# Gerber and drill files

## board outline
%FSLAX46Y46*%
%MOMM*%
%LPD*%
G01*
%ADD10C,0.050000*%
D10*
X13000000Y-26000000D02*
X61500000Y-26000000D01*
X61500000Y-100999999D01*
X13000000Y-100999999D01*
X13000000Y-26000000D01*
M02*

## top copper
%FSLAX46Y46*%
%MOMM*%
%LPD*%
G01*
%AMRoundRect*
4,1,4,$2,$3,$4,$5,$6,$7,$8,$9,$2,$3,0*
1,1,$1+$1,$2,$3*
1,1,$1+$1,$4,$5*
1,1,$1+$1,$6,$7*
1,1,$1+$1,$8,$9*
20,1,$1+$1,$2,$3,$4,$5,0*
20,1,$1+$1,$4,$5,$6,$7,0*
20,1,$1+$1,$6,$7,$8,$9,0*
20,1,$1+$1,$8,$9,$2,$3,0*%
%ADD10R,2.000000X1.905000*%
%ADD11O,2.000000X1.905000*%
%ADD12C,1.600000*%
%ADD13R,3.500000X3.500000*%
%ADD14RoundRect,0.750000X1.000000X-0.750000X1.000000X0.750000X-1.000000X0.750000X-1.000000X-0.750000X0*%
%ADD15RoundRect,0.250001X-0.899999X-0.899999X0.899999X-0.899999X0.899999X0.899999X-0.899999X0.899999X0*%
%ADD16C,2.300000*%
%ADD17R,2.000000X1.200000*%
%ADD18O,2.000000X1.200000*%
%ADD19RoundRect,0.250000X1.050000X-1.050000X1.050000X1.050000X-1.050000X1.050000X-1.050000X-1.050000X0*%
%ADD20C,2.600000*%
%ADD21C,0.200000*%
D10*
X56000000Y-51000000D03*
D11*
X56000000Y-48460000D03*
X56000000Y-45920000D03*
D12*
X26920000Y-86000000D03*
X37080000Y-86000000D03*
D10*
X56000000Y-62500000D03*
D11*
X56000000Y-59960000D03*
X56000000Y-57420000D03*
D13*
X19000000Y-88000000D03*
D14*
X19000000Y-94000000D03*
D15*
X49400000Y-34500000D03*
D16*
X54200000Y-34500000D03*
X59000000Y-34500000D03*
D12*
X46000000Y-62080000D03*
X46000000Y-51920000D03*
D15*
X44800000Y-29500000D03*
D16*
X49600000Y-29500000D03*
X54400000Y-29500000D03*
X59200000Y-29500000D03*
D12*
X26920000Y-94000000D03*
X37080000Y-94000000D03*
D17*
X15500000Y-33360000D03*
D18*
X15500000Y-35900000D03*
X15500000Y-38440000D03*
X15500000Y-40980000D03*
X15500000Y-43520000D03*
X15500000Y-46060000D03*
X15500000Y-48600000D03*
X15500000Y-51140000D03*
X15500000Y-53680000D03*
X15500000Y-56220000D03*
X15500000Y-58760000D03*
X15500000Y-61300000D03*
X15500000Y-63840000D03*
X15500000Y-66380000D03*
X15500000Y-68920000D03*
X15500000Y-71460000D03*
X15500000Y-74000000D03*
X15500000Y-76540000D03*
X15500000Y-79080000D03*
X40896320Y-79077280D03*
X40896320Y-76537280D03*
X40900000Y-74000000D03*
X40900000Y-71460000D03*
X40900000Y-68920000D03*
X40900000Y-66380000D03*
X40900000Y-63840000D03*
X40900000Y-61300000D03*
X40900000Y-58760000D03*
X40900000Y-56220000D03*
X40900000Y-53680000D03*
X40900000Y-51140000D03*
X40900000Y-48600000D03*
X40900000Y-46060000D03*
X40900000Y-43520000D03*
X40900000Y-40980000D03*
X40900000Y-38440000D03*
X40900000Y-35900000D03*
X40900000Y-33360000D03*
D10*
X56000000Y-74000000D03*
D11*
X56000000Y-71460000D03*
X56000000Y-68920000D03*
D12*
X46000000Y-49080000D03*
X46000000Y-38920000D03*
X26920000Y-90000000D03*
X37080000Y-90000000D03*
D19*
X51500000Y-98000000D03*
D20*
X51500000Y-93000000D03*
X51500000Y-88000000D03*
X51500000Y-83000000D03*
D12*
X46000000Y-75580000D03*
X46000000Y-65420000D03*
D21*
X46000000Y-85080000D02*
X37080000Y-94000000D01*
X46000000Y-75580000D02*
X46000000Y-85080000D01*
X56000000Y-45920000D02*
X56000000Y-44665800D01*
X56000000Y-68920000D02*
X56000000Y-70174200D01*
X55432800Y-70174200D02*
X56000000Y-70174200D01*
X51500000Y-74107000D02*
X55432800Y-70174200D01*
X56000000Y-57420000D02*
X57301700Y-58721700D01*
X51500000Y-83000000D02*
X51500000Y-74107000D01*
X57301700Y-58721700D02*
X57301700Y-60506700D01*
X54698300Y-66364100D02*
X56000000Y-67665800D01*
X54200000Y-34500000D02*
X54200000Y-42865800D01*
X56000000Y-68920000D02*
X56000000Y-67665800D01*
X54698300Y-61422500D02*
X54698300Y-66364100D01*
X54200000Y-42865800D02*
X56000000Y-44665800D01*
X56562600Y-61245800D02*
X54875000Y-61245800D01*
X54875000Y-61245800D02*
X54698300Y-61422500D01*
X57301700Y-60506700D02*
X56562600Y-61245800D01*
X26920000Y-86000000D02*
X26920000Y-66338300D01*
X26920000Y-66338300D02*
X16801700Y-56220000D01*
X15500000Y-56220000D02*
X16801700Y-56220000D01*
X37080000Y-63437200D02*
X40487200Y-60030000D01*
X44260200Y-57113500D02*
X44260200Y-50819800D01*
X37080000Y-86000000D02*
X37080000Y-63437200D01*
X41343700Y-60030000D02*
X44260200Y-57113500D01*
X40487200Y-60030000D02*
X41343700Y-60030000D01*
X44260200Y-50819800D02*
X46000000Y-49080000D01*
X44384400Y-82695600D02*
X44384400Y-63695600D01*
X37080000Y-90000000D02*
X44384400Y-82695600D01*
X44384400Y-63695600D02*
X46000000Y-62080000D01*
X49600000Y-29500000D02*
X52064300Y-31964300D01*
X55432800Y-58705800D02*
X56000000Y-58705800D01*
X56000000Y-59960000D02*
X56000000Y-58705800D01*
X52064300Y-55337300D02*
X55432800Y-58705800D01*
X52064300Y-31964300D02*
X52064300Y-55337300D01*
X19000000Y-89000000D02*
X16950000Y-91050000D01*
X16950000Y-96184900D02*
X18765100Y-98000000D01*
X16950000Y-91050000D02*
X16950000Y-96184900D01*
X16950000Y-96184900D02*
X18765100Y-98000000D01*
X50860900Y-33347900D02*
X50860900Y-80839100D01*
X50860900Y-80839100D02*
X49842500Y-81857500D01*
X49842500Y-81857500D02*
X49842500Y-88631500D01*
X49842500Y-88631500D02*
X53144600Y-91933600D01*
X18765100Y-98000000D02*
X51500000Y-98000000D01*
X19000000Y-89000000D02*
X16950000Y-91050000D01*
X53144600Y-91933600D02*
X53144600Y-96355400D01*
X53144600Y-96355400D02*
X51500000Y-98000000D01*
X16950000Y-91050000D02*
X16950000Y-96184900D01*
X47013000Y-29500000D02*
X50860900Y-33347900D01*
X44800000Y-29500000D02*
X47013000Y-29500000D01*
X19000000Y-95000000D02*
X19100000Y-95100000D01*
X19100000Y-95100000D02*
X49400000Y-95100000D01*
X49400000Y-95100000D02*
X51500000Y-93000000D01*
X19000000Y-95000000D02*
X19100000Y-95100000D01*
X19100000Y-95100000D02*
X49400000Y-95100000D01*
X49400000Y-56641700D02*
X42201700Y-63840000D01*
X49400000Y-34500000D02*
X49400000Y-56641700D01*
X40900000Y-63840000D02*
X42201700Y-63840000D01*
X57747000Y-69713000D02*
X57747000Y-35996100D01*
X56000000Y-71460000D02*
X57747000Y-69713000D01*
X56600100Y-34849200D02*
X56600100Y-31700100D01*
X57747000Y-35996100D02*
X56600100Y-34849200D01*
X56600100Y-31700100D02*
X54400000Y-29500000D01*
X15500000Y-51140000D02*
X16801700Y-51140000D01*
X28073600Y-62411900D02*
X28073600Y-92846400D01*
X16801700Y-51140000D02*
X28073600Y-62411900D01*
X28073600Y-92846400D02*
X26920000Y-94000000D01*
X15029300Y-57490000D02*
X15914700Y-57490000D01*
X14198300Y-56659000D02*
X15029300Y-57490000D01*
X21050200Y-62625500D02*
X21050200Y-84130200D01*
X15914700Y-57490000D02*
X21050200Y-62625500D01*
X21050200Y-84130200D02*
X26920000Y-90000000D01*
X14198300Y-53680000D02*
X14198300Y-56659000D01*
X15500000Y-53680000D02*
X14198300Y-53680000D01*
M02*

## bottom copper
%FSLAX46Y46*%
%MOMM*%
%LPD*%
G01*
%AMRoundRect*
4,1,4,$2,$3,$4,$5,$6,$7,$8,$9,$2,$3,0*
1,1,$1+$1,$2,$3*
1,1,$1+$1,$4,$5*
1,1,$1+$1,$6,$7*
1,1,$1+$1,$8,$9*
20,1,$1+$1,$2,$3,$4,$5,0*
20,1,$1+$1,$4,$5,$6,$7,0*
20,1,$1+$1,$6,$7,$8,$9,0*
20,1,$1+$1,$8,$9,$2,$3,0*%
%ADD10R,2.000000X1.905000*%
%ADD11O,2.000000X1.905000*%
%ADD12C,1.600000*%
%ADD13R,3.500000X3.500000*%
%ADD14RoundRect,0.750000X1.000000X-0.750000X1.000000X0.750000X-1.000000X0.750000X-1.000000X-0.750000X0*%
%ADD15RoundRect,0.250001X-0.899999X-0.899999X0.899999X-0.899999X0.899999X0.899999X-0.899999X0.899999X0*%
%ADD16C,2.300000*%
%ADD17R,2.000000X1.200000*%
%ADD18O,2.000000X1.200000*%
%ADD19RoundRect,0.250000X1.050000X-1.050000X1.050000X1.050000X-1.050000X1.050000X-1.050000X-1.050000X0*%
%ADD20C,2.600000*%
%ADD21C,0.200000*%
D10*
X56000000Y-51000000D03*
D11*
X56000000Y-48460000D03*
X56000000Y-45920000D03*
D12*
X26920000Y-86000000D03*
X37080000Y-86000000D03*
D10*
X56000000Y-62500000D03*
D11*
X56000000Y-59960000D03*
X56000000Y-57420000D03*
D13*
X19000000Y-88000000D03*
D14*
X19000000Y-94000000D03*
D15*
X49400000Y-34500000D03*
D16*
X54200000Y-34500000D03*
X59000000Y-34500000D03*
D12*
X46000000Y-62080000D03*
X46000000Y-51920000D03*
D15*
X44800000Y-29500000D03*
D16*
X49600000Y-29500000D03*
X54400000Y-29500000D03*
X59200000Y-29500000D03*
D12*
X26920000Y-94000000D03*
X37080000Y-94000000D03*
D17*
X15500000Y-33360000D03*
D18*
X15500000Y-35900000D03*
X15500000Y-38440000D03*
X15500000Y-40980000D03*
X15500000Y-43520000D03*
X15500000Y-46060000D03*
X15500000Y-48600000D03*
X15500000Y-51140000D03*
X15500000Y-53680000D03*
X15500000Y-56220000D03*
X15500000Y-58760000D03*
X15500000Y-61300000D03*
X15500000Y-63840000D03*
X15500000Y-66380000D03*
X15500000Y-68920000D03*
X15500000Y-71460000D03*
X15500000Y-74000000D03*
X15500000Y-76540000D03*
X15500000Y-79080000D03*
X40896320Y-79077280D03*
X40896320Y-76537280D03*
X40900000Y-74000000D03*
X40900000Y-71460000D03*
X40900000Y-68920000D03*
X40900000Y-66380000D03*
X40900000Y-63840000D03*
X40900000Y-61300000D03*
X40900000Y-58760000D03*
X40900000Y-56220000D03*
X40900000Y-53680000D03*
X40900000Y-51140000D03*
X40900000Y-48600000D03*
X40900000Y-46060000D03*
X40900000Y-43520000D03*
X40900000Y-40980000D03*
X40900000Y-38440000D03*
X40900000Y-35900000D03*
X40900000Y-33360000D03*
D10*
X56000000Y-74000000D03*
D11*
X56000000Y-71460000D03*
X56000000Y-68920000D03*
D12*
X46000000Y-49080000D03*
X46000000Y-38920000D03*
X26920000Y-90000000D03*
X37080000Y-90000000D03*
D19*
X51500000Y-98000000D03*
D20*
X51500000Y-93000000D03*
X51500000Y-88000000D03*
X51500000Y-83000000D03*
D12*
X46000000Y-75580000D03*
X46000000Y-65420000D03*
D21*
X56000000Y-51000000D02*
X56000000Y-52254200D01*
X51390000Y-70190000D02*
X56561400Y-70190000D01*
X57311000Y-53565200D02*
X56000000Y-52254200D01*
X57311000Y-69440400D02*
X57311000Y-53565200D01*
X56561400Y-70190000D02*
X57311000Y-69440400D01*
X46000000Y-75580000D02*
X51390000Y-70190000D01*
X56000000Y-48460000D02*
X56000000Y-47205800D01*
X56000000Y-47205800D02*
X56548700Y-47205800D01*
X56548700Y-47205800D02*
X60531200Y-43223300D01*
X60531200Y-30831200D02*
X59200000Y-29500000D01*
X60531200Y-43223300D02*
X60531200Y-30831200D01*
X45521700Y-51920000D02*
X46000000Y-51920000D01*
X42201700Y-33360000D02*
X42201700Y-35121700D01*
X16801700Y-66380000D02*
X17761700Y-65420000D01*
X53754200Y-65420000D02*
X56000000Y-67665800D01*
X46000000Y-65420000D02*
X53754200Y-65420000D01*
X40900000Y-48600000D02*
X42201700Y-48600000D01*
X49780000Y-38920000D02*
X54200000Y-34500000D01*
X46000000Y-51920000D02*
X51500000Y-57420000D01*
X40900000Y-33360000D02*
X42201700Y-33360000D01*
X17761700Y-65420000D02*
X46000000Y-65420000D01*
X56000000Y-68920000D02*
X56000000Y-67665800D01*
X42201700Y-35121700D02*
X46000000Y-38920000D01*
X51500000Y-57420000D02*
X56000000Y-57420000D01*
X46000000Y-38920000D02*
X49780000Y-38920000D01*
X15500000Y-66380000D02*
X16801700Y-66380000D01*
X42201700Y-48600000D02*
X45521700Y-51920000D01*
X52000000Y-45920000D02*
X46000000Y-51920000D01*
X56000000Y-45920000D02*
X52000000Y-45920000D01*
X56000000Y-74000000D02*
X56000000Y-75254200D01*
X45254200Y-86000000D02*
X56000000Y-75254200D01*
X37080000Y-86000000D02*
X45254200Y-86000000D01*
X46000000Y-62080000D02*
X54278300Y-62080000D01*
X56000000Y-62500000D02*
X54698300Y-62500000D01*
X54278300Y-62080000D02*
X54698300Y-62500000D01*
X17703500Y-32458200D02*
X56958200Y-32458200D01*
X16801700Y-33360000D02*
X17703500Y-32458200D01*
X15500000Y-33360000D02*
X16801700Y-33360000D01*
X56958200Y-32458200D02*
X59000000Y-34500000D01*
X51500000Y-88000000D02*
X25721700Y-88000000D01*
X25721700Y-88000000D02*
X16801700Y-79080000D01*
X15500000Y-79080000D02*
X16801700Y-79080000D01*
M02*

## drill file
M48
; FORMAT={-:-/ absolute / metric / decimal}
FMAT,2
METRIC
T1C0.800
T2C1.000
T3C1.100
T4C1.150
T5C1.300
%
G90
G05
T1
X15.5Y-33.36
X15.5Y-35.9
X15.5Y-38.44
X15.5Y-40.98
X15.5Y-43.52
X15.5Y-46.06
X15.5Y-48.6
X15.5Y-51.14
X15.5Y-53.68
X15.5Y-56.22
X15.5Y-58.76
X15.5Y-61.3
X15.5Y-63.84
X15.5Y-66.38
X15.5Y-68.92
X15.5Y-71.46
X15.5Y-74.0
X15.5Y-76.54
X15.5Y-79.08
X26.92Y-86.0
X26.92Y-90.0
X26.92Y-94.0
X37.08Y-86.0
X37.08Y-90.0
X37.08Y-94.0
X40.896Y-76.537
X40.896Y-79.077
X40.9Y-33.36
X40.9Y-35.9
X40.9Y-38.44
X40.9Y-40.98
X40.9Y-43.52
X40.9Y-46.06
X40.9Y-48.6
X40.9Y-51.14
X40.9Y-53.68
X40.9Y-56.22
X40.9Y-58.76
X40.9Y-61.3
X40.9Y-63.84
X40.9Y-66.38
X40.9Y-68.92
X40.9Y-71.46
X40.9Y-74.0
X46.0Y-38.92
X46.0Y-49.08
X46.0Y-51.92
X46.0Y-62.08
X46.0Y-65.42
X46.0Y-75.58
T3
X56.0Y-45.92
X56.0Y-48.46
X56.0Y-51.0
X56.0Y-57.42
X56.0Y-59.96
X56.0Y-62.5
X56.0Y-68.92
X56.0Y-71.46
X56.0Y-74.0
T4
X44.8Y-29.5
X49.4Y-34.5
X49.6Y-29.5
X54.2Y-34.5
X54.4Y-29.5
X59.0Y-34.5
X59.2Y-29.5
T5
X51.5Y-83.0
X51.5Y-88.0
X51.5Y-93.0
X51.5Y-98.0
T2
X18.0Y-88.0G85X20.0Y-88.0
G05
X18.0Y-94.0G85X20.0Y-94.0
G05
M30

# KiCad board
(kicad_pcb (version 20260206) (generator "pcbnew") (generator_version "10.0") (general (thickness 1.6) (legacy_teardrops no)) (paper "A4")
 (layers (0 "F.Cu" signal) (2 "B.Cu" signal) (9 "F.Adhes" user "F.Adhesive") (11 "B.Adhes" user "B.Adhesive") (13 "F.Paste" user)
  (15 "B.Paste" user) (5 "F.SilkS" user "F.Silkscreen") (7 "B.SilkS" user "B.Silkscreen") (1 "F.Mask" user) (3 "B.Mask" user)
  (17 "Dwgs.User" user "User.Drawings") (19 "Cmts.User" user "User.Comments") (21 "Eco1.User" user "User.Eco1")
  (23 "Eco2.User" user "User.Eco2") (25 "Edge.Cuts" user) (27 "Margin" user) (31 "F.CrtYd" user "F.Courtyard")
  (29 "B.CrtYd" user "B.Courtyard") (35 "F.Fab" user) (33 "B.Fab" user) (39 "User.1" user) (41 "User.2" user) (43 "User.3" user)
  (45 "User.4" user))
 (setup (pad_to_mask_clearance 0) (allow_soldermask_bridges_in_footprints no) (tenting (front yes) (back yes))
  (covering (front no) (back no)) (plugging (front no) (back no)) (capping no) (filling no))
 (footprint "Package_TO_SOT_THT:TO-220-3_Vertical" (layer "F.Cu") (at 56 51 90)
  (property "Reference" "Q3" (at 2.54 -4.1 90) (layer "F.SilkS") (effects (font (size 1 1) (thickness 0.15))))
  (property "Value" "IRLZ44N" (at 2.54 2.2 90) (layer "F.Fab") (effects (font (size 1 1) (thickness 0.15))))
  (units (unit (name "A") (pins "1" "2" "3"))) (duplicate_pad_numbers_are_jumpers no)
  (pad "1" thru_hole rect (at 0 0 90) (size 1.905 2) (drill 1.1) (layers "*.Cu" "*.Mask") (remove_unused_layers no) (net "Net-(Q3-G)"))
  (pad "2" thru_hole oval (at 2.54 0 90) (size 1.905 2) (drill 1.1) (layers "*.Cu" "*.Mask") (remove_unused_layers no) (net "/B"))
  (pad "3" thru_hole oval (at 5.08 0 90) (size 1.905 2) (drill 1.1) (layers "*.Cu" "*.Mask") (remove_unused_layers no) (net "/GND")))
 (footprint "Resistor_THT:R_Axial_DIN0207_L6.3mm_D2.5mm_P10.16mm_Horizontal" (layer "F.Cu") (at 26.92 86)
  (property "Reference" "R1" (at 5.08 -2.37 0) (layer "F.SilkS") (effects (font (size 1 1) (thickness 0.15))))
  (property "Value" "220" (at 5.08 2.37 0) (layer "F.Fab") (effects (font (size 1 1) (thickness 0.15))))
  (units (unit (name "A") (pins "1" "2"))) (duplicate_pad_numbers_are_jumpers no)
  (pad "1" thru_hole circle (at 0 0) (size 1.6 1.6) (drill 0.8) (layers "*.Cu" "*.Mask") (remove_unused_layers no)
   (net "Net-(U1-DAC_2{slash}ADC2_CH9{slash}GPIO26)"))
  (pad "2" thru_hole circle (at 10.16 0) (size 1.6 1.6) (drill 0.8) (layers "*.Cu" "*.Mask") (remove_unused_layers no) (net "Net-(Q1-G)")))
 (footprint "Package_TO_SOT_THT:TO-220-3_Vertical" (layer "F.Cu") (at 56 62.5 90)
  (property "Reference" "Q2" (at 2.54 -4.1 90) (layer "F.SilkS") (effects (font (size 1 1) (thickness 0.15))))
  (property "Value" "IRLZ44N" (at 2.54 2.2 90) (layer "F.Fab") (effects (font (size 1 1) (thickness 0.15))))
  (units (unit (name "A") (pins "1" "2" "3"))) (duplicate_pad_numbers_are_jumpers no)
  (pad "1" thru_hole rect (at 0 0 90) (size 1.905 2) (drill 1.1) (layers "*.Cu" "*.Mask") (remove_unused_layers no) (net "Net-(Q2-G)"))
  (pad "2" thru_hole oval (at 2.54 0 90) (size 1.905 2) (drill 1.1) (layers "*.Cu" "*.Mask") (remove_unused_layers no) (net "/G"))
  (pad "3" thru_hole oval (at 5.08 0 90) (size 1.905 2) (drill 1.1) (layers "*.Cu" "*.Mask") (remove_unused_layers no) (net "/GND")))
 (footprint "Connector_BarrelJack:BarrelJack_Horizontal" (layer "F.Cu") (at 19 88 90)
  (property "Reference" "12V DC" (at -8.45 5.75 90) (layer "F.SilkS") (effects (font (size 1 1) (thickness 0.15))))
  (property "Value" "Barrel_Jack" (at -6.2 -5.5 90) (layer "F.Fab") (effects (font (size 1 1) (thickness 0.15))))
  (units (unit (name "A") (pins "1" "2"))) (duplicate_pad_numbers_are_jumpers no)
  (pad "1" thru_hole rect (at 0 0 90) (size 3.5 3.5) (drill oval 1 3) (layers "*.Cu" "*.Mask") (remove_unused_layers no) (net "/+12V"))
  (pad "2" thru_hole roundrect (at -6 0 90) (size 3 3.5) (drill oval 1 3) (layers "*.Cu" "*.Mask") (remove_unused_layers no)
   (roundrect_rratio 0.25) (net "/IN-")))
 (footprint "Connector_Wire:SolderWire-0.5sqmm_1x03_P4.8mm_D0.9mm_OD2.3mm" (layer "F.Cu") (at 49.4 34.5)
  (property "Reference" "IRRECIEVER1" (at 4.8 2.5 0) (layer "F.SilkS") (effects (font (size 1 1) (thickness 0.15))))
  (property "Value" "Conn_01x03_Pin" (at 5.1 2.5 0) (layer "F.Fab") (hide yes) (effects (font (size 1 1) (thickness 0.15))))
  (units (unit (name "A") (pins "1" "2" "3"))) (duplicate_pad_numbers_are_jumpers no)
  (pad "1" thru_hole roundrect (at 0 0) (size 2.3 2.3) (drill 1.15) (layers "*.Cu" "*.Mask") (remove_unused_layers no)
   (roundrect_rratio 0.108696) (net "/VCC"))
  (pad "2" thru_hole circle (at 4.8 0) (size 2.3 2.3) (drill 1.15) (layers "*.Cu" "*.Mask") (remove_unused_layers no) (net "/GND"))
  (pad "3" thru_hole circle (at 9.6 0) (size 2.3 2.3) (drill 1.15) (layers "*.Cu" "*.Mask") (remove_unused_layers no) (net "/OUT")))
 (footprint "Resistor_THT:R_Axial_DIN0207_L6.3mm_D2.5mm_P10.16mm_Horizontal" (layer "F.Cu") (at 46 62.08 90)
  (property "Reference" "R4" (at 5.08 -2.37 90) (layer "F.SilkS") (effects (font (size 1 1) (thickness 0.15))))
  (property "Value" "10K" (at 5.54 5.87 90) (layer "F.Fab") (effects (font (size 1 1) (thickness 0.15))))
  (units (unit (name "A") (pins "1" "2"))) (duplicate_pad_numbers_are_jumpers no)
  (pad "1" thru_hole circle (at 0 0 90) (size 1.6 1.6) (drill 0.8) (layers "*.Cu" "*.Mask") (remove_unused_layers no) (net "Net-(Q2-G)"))
  (pad "2" thru_hole circle (at 10.16 0 90) (size 1.6 1.6) (drill 0.8) (layers "*.Cu" "*.Mask") (remove_unused_layers no) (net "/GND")))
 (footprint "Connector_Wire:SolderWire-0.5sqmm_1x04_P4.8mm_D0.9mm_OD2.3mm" (layer "F.Cu") (at 44.8 29.5)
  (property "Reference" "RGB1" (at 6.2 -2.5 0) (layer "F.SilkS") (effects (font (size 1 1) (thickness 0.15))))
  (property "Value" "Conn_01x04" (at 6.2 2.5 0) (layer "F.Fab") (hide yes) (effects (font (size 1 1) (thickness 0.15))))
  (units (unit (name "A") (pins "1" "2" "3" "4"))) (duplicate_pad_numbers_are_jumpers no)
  (pad "1" thru_hole roundrect (at 0 0) (size 2.3 2.3) (drill 1.15) (layers "*.Cu" "*.Mask") (remove_unused_layers no)
   (roundrect_rratio 0.108696) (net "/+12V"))
  (pad "2" thru_hole circle (at 4.8 0) (size 2.3 2.3) (drill 1.15) (layers "*.Cu" "*.Mask") (remove_unused_layers no) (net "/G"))
  (pad "3" thru_hole circle (at 9.6 0) (size 2.3 2.3) (drill 1.15) (layers "*.Cu" "*.Mask") (remove_unused_layers no) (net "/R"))
  (pad "4" thru_hole circle (at 14.4 0) (size 2.3 2.3) (drill 1.15) (layers "*.Cu" "*.Mask") (remove_unused_layers no) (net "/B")))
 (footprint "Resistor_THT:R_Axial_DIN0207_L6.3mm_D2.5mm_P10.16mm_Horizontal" (layer "F.Cu") (at 26.92 94)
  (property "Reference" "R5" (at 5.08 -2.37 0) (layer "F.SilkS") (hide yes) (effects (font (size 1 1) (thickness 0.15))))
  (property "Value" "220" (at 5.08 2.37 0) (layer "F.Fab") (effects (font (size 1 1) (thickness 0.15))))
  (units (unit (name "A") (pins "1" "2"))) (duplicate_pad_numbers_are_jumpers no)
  (pad "1" thru_hole circle (at 0 0) (size 1.6 1.6) (drill 0.8) (layers "*.Cu" "*.Mask") (remove_unused_layers no)
   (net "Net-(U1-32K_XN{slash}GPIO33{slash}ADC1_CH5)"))
  (pad "2" thru_hole circle (at 10.16 0) (size 1.6 1.6) (drill 0.8) (layers "*.Cu" "*.Mask") (remove_unused_layers no) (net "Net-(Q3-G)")))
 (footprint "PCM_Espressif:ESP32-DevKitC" (layer "F.Cu") (at 15.5 33.36)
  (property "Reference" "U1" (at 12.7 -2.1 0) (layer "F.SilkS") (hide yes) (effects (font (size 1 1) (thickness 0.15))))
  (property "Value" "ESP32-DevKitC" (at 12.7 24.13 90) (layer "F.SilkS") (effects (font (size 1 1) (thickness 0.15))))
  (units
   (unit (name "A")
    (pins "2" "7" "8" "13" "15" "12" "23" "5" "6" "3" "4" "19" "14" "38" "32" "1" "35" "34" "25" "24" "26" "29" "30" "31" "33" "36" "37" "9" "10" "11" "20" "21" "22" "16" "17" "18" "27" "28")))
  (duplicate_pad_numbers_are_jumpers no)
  (pad "1" thru_hole rect (at 0 0 270) (size 1.2 2) (drill 0.8) (layers "*.Cu" "*.Mask") (remove_unused_layers no) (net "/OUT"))
  (pad "2" thru_hole oval (at 0 2.54 270) (size 1.2 2) (drill 0.8) (layers "*.Cu" "*.Mask") (remove_unused_layers no)
   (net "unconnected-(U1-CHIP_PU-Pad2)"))
  (pad "3" thru_hole oval (at 0 5.08 270) (size 1.2 2) (drill 0.8) (layers "*.Cu" "*.Mask") (remove_unused_layers no)
   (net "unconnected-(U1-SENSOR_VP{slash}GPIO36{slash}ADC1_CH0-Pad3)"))
  (pad "4" thru_hole oval (at 0 7.62 270) (size 1.2 2) (drill 0.8) (layers "*.Cu" "*.Mask") (remove_unused_layers no)
   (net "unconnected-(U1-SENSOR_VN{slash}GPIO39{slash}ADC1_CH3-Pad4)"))
  (pad "5" thru_hole oval (at 0 10.16 270) (size 1.2 2) (drill 0.8) (layers "*.Cu" "*.Mask") (remove_unused_layers no)
   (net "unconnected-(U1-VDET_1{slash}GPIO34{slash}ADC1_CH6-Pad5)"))
  (pad "6" thru_hole oval (at 0 12.7 270) (size 1.2 2) (drill 0.8) (layers "*.Cu" "*.Mask") (remove_unused_layers no)
   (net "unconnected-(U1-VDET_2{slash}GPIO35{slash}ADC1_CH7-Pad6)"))
  (pad "7" thru_hole oval (at 0 15.24 270) (size 1.2 2) (drill 0.8) (layers "*.Cu" "*.Mask") (remove_unused_layers no)
   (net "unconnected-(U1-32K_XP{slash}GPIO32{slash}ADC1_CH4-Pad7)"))
  (pad "8" thru_hole oval (at 0 17.78 270) (size 1.2 2) (drill 0.8) (layers "*.Cu" "*.Mask") (remove_unused_layers no)
   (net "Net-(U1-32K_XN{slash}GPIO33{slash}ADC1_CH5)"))
  (pad "9" thru_hole oval (at 0 20.32 270) (size 1.2 2) (drill 0.8) (layers "*.Cu" "*.Mask") (remove_unused_layers no)
   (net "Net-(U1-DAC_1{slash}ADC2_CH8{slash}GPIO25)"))
  (pad "10" thru_hole oval (at 0 22.86 270) (size 1.2 2) (drill 0.8) (layers "*.Cu" "*.Mask") (remove_unused_layers no)
   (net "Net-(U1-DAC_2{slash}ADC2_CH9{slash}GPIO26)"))
  (pad "11" thru_hole oval (at 0 25.4 270) (size 1.2 2) (drill 0.8) (layers "*.Cu" "*.Mask") (remove_unused_layers no)
   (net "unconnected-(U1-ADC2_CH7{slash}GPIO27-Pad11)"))
  (pad "12" thru_hole oval (at 0 27.94 270) (size 1.2 2) (drill 0.8) (layers "*.Cu" "*.Mask") (remove_unused_layers no)
   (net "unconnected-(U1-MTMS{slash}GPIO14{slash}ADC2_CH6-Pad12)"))
  (pad "13" thru_hole oval (at 0 30.48 270) (size 1.2 2) (drill 0.8) (layers "*.Cu" "*.Mask") (remove_unused_layers no)
   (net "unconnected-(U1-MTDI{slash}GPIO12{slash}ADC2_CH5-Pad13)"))
  (pad "14" thru_hole oval (at 0 33.02 270) (size 1.2 2) (drill 0.8) (layers "*.Cu" "*.Mask") (remove_unused_layers no) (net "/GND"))
  (pad "15" thru_hole oval (at 0 35.56 270) (size 1.2 2) (drill 0.8) (layers "*.Cu" "*.Mask") (remove_unused_layers no)
   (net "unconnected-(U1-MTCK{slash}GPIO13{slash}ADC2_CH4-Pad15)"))
  (pad "16" thru_hole oval (at 0 38.1 270) (size 1.2 2) (drill 0.8) (layers "*.Cu" "*.Mask") (remove_unused_layers no)
   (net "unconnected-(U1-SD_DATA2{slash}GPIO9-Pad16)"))
  (pad "17" thru_hole oval (at 0 40.64 270) (size 1.2 2) (drill 0.8) (layers "*.Cu" "*.Mask") (remove_unused_layers no)
   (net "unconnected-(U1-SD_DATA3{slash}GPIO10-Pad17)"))
  (pad "18" thru_hole oval (at 0 43.18 270) (size 1.2 2) (drill 0.8) (layers "*.Cu" "*.Mask") (remove_unused_layers no)
   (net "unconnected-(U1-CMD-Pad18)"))
  (pad "19" thru_hole oval (at 0 45.72 270) (size 1.2 2) (drill 0.8) (layers "*.Cu" "*.Mask") (remove_unused_layers no) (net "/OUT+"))
  (pad "20" thru_hole oval (at 25.39632 45.71728 270) (size 1.2 2) (drill 0.8) (layers "*.Cu" "*.Mask") (remove_unused_layers no)
   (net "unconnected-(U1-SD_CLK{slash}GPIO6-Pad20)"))
  (pad "21" thru_hole oval (at 25.39632 43.17728 270) (size 1.2 2) (drill 0.8) (layers "*.Cu" "*.Mask") (remove_unused_layers no)
   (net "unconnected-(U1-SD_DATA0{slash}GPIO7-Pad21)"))
  (pad "22" thru_hole oval (at 25.4 40.64 270) (size 1.2 2) (drill 0.8) (layers "*.Cu" "*.Mask") (remove_unused_layers no)
   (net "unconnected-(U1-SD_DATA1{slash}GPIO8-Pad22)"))
  (pad "23" thru_hole oval (at 25.4 38.1 270) (size 1.2 2) (drill 0.8) (layers "*.Cu" "*.Mask") (remove_unused_layers no)
   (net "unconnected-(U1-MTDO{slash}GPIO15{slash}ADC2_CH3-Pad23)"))
  (pad "24" thru_hole oval (at 25.4 35.56 270) (size 1.2 2) (drill 0.8) (layers "*.Cu" "*.Mask") (remove_unused_layers no)
   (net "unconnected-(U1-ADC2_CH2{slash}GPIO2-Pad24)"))
  (pad "25" thru_hole oval (at 25.4 33.02 270) (size 1.2 2) (drill 0.8) (layers "*.Cu" "*.Mask") (remove_unused_layers no)
   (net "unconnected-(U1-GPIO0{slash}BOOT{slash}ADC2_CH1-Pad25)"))
  (pad "26" thru_hole oval (at 25.4 30.48 270) (size 1.2 2) (drill 0.8) (layers "*.Cu" "*.Mask") (remove_unused_layers no) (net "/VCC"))
  (pad "27" thru_hole oval (at 25.4 27.94 270) (size 1.2 2) (drill 0.8) (layers "*.Cu" "*.Mask") (remove_unused_layers no)
   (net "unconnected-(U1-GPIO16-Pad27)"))
  (pad "28" thru_hole oval (at 25.4 25.4 270) (size 1.2 2) (drill 0.8) (layers "*.Cu" "*.Mask") (remove_unused_layers no)
   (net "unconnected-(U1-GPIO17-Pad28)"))
  (pad "29" thru_hole oval (at 25.4 22.86 270) (size 1.2 2) (drill 0.8) (layers "*.Cu" "*.Mask") (remove_unused_layers no)
   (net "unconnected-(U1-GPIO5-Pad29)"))
  (pad "30" thru_hole oval (at 25.4 20.32 270) (size 1.2 2) (drill 0.8) (layers "*.Cu" "*.Mask") (remove_unused_layers no)
   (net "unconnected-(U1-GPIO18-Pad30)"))
  (pad "31" thru_hole oval (at 25.4 17.78 270) (size 1.2 2) (drill 0.8) (layers "*.Cu" "*.Mask") (remove_unused_layers no)
   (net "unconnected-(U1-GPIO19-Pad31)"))
  (pad "32" thru_hole oval (at 25.4 15.24 270) (size 1.2 2) (drill 0.8) (layers "*.Cu" "*.Mask") (remove_unused_layers no) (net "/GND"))
  (pad "33" thru_hole oval (at 25.4 12.7 270) (size 1.2 2) (drill 0.8) (layers "*.Cu" "*.Mask") (remove_unused_layers no)
   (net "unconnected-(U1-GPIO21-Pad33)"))
  (pad "34" thru_hole oval (at 25.4 10.16 270) (size 1.2 2) (drill 0.8) (layers "*.Cu" "*.Mask") (remove_unused_layers no)
   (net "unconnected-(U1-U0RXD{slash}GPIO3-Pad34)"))
  (pad "35" thru_hole oval (at 25.4 7.62 270) (size 1.2 2) (drill 0.8) (layers "*.Cu" "*.Mask") (remove_unused_layers no)
   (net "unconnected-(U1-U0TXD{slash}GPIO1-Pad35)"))
  (pad "36" thru_hole oval (at 25.4 5.08 270) (size 1.2 2) (drill 0.8) (layers "*.Cu" "*.Mask") (remove_unused_layers no)
   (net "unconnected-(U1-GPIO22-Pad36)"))
  (pad "37" thru_hole oval (at 25.4 2.54 270) (size 1.2 2) (drill 0.8) (layers "*.Cu" "*.Mask") (remove_unused_layers no)
   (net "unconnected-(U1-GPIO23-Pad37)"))
  (pad "38" thru_hole oval (at 25.4 0 270) (size 1.2 2) (drill 0.8) (layers "*.Cu" "*.Mask") (remove_unused_layers no) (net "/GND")))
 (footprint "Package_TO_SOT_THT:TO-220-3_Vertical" (layer "F.Cu") (at 56 74 90)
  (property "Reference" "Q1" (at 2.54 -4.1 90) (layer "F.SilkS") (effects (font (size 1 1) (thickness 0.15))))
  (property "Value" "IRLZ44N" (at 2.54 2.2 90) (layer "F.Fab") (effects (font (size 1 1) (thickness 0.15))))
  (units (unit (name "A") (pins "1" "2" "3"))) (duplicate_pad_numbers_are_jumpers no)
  (pad "1" thru_hole rect (at 0 0 90) (size 1.905 2) (drill 1.1) (layers "*.Cu" "*.Mask") (remove_unused_layers no) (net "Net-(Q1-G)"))
  (pad "2" thru_hole oval (at 2.54 0 90) (size 1.905 2) (drill 1.1) (layers "*.Cu" "*.Mask") (remove_unused_layers no) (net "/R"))
  (pad "3" thru_hole oval (at 5.08 0 90) (size 1.905 2) (drill 1.1) (layers "*.Cu" "*.Mask") (remove_unused_layers no) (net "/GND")))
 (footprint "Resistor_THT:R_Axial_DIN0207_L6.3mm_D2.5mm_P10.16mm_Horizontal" (layer "F.Cu") (at 46 49.08 90)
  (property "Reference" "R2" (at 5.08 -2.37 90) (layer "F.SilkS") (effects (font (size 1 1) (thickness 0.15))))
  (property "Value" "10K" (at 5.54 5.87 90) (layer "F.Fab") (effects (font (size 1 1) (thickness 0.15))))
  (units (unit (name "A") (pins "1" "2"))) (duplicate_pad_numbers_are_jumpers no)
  (pad "1" thru_hole circle (at 0 0 90) (size 1.6 1.6) (drill 0.8) (layers "*.Cu" "*.Mask") (remove_unused_layers no) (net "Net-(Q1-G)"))
  (pad "2" thru_hole circle (at 10.16 0 90) (size 1.6 1.6) (drill 0.8) (layers "*.Cu" "*.Mask") (remove_unused_layers no) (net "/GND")))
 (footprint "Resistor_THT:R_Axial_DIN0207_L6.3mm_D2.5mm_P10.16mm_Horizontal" (layer "F.Cu") (at 26.92 90)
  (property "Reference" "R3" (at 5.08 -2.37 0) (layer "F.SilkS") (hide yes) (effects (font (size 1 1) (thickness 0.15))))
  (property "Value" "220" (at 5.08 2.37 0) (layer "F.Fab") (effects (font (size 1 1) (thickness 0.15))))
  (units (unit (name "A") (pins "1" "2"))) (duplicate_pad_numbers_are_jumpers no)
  (pad "1" thru_hole circle (at 0 0) (size 1.6 1.6) (drill 0.8) (layers "*.Cu" "*.Mask") (remove_unused_layers no)
   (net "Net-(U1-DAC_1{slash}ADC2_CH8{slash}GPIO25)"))
  (pad "2" thru_hole circle (at 10.16 0) (size 1.6 1.6) (drill 0.8) (layers "*.Cu" "*.Mask") (remove_unused_layers no) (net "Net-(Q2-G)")))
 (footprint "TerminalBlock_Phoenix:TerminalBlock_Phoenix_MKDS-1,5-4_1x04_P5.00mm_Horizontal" (layer "F.Cu") (at 51.5 98 90)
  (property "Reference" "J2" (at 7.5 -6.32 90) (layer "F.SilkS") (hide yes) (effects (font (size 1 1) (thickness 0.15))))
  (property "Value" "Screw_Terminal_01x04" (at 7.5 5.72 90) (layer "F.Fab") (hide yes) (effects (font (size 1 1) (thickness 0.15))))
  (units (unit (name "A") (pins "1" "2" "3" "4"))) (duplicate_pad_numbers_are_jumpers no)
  (pad "1" thru_hole roundrect (at 0 0 90) (size 2.6 2.6) (drill 1.3) (layers "*.Cu" "*.Mask") (remove_unused_layers no)
   (roundrect_rratio 0.096154) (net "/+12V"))
  (pad "2" thru_hole circle (at 5 0 90) (size 2.6 2.6) (drill 1.3) (layers "*.Cu" "*.Mask") (remove_unused_layers no) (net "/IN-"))
  (pad "3" thru_hole circle (at 10 0 90) (size 2.6 2.6) (drill 1.3) (layers "*.Cu" "*.Mask") (remove_unused_layers no) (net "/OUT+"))
  (pad "4" thru_hole circle (at 15 0 90) (size 2.6 2.6) (drill 1.3) (layers "*.Cu" "*.Mask") (remove_unused_layers no) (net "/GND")))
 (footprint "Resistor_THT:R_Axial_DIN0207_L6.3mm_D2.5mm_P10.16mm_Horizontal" (layer "F.Cu") (at 46 75.58 90)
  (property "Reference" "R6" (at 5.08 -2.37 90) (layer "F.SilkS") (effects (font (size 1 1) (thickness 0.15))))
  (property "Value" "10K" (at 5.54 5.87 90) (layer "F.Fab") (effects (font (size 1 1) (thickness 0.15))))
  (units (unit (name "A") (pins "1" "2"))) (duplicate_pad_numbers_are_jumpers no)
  (pad "1" thru_hole circle (at 0 0 90) (size 1.6 1.6) (drill 0.8) (layers "*.Cu" "*.Mask") (remove_unused_layers no) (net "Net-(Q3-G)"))
  (pad "2" thru_hole circle (at 10.16 0 90) (size 1.6 1.6) (drill 0.8) (layers "*.Cu" "*.Mask") (remove_unused_layers no) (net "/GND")))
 (gr_rect (start 13 26) (end 61.5 100.999999) (stroke (width 0.05) (type default)) (fill no) (layer "Edge.Cuts"))
 (segment (start 46 85.08) (end 37.08 94) (width 0.2) (layer "F.Cu") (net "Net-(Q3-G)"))
 (segment (start 46 75.58) (end 46 85.08) (width 0.2) (layer "F.Cu") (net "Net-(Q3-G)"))
 (segment (start 56 51) (end 56 52.2542) (width 0.2) (layer "B.Cu") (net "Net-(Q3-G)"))
 (segment (start 51.39 70.19) (end 56.5614 70.19) (width 0.2) (layer "B.Cu") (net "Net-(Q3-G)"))
 (segment (start 57.311 53.5652) (end 56 52.2542) (width 0.2) (layer "B.Cu") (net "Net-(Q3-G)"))
 (segment (start 57.311 69.4404) (end 57.311 53.5652) (width 0.2) (layer "B.Cu") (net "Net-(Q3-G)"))
 (segment (start 56.5614 70.19) (end 57.311 69.4404) (width 0.2) (layer "B.Cu") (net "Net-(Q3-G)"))
 (segment (start 46 75.58) (end 51.39 70.19) (width 0.2) (layer "B.Cu") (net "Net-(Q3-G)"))
 (segment (start 56 48.46) (end 56 47.2058) (width 0.2) (layer "B.Cu") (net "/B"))
 (segment (start 56 47.2058) (end 56.5487 47.2058) (width 0.2) (layer "B.Cu") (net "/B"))
 (segment (start 56.5487 47.2058) (end 60.5312 43.2233) (width 0.2) (layer "B.Cu") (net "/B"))
 (segment (start 60.5312 30.8312) (end 59.2 29.5) (width 0.2) (layer "B.Cu") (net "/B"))
 (segment (start 60.5312 43.2233) (end 60.5312 30.8312) (width 0.2) (layer "B.Cu") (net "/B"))
 (segment (start 56 45.92) (end 56 44.6658) (width 0.2) (layer "F.Cu") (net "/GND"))
 (segment (start 56 68.92) (end 56 70.1742) (width 0.2) (layer "F.Cu") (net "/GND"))
 (segment (start 55.4328 70.1742) (end 56 70.1742) (width 0.2) (layer "F.Cu") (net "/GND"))
 (segment (start 51.5 74.107) (end 55.4328 70.1742) (width 0.2) (layer "F.Cu") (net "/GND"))
 (segment (start 56 57.42) (end 57.3017 58.7217) (width 0.2) (layer "F.Cu") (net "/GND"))
 (segment (start 51.5 83) (end 51.5 74.107) (width 0.2) (layer "F.Cu") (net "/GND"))
 (segment (start 57.3017 58.7217) (end 57.3017 60.5067) (width 0.2) (layer "F.Cu") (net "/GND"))
 (segment (start 54.6983 66.3641) (end 56 67.6658) (width 0.2) (layer "F.Cu") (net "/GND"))
 (segment (start 54.2 34.5) (end 54.2 42.8658) (width 0.2) (layer "F.Cu") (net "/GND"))
 (segment (start 56 68.92) (end 56 67.6658) (width 0.2) (layer "F.Cu") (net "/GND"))
 (segment (start 54.6983 61.4225) (end 54.6983 66.3641) (width 0.2) (layer "F.Cu") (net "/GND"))
 (segment (start 54.2 42.8658) (end 56 44.6658) (width 0.2) (layer "F.Cu") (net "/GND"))
 (segment (start 56.5626 61.2458) (end 54.875 61.2458) (width 0.2) (layer "F.Cu") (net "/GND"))
 (segment (start 54.875 61.2458) (end 54.6983 61.4225) (width 0.2) (layer "F.Cu") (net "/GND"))
 (segment (start 57.3017 60.5067) (end 56.5626 61.2458) (width 0.2) (layer "F.Cu") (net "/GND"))
 (segment (start 45.5217 51.92) (end 46 51.92) (width 0.2) (layer "B.Cu") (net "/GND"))
 (segment (start 42.2017 33.36) (end 42.2017 35.1217) (width 0.2) (layer "B.Cu") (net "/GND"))
 (segment (start 16.8017 66.38) (end 17.7617 65.42) (width 0.2) (layer "B.Cu") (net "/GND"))
 (segment (start 53.7542 65.42) (end 56 67.6658) (width 0.2) (layer "B.Cu") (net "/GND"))
 (segment (start 46 65.42) (end 53.7542 65.42) (width 0.2) (layer "B.Cu") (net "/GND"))
 (segment (start 40.9 48.6) (end 42.2017 48.6) (width 0.2) (layer "B.Cu") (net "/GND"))
 (segment (start 49.78 38.92) (end 54.2 34.5) (width 0.2) (layer "B.Cu") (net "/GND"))
 (segment (start 46 51.92) (end 51.5 57.42) (width 0.2) (layer "B.Cu") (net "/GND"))
 (segment (start 40.9 33.36) (end 42.2017 33.36) (width 0.2) (layer "B.Cu") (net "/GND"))
 (segment (start 17.7617 65.42) (end 46 65.42) (width 0.2) (layer "B.Cu") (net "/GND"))
 (segment (start 56 68.92) (end 56 67.6658) (width 0.2) (layer "B.Cu") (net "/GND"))
 (segment (start 42.2017 35.1217) (end 46 38.92) (width 0.2) (layer "B.Cu") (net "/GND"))
 (segment (start 51.5 57.42) (end 56 57.42) (width 0.2) (layer "B.Cu") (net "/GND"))
 (segment (start 46 38.92) (end 49.78 38.92) (width 0.2) (layer "B.Cu") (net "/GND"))
 (segment (start 15.5 66.38) (end 16.8017 66.38) (width 0.2) (layer "B.Cu") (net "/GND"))
 (segment (start 42.2017 48.6) (end 45.5217 51.92) (width 0.2) (layer "B.Cu") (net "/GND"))
 (segment (start 52 45.92) (end 46 51.92) (width 0.2) (layer "B.Cu") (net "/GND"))
 (segment (start 56 45.92) (end 52 45.92) (width 0.2) (layer "B.Cu") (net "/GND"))
 (segment (start 26.92 86) (end 26.92 66.3383) (width 0.2) (layer "F.Cu") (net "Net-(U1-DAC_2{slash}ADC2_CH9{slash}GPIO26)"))
 (segment (start 26.92 66.3383) (end 16.8017 56.22) (width 0.2) (layer "F.Cu") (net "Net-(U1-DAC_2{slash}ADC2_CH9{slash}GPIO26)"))
 (segment (start 15.5 56.22) (end 16.8017 56.22) (width 0.2) (layer "F.Cu") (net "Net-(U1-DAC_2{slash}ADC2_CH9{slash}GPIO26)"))
 (segment (start 37.08 63.4372) (end 40.4872 60.03) (width 0.2) (layer "F.Cu") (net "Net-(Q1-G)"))
 (segment (start 44.2602 57.1135) (end 44.2602 50.8198) (width 0.2) (layer "F.Cu") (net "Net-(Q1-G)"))
 (segment (start 37.08 86) (end 37.08 63.4372) (width 0.2) (layer "F.Cu") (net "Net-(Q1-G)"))
 (segment (start 41.3437 60.03) (end 44.2602 57.1135) (width 0.2) (layer "F.Cu") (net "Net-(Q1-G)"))
 (segment (start 40.4872 60.03) (end 41.3437 60.03) (width 0.2) (layer "F.Cu") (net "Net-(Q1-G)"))
 (segment (start 44.2602 50.8198) (end 46 49.08) (width 0.2) (layer "F.Cu") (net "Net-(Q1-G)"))
 (segment (start 56 74) (end 56 75.2542) (width 0.2) (layer "B.Cu") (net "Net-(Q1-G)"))
 (segment (start 45.2542 86) (end 56 75.2542) (width 0.2) (layer "B.Cu") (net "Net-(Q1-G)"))
 (segment (start 37.08 86) (end 45.2542 86) (width 0.2) (layer "B.Cu") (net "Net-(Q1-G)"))
 (segment (start 44.3844 82.6956) (end 44.3844 63.6956) (width 0.2) (layer "F.Cu") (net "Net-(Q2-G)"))
 (segment (start 37.08 90) (end 44.3844 82.6956) (width 0.2) (layer "F.Cu") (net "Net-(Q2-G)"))
 (segment (start 44.3844 63.6956) (end 46 62.08) (width 0.2) (layer "F.Cu") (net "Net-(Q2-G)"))
 (segment (start 46 62.08) (end 54.2783 62.08) (width 0.2) (layer "B.Cu") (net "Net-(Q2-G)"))
 (segment (start 56 62.5) (end 54.6983 62.5) (width 0.2) (layer "B.Cu") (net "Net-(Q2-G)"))
 (segment (start 54.2783 62.08) (end 54.6983 62.5) (width 0.2) (layer "B.Cu") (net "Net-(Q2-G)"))
 (segment (start 49.6 29.5) (end 52.0643 31.9643) (width 0.2) (layer "F.Cu") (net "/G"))
 (segment (start 55.4328 58.7058) (end 56 58.7058) (width 0.2) (layer "F.Cu") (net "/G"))
 (segment (start 56 59.96) (end 56 58.7058) (width 0.2) (layer "F.Cu") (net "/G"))
 (segment (start 52.0643 55.3373) (end 55.4328 58.7058) (width 0.2) (layer "F.Cu") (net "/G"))
 (segment (start 52.0643 31.9643) (end 52.0643 55.3373) (width 0.2) (layer "F.Cu") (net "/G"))
 (segment (start 19 89) (end 16.95 91.05) (width 0.2) (layer "F.Cu") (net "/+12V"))
 (segment (start 16.95 96.1849) (end 18.7651 98) (width 0.2) (layer "F.Cu") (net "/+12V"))
 (segment (start 16.95 91.05) (end 16.95 96.1849) (width 0.2) (layer "F.Cu") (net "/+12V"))
 (segment (start 16.95 96.1849) (end 18.7651 98) (width 0.2) (layer "F.Cu") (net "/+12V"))
 (segment (start 50.8609 33.3479) (end 50.8609 80.8391) (width 0.2) (layer "F.Cu") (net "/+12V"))
 (segment (start 50.8609 80.8391) (end 49.8425 81.8575) (width 0.2) (layer "F.Cu") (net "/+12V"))
 (segment (start 49.8425 81.8575) (end 49.8425 88.6315) (width 0.2) (layer "F.Cu") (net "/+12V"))
 (segment (start 49.8425 88.6315) (end 53.1446 91.9336) (width 0.2) (layer "F.Cu") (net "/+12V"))
 (segment (start 18.7651 98) (end 51.5 98) (width 0.2) (layer "F.Cu") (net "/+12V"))
 (segment (start 19 89) (end 16.95 91.05) (width 0.2) (layer "F.Cu") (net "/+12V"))
 (segment (start 53.1446 91.9336) (end 53.1446 96.3554) (width 0.2) (layer "F.Cu") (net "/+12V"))
 (segment (start 53.1446 96.3554) (end 51.5 98) (width 0.2) (layer "F.Cu") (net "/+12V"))
 (segment (start 16.95 91.05) (end 16.95 96.1849) (width 0.2) (layer "F.Cu") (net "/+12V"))
 (segment (start 47.013 29.5) (end 50.8609 33.3479) (width 0.2) (layer "F.Cu") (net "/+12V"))
 (segment (start 44.8 29.5) (end 47.013 29.5) (width 0.2) (layer "F.Cu") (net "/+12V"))
 (segment (start 19 95) (end 19.1 95.1) (width 0.2) (layer "F.Cu") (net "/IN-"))
 (segment (start 19.1 95.1) (end 49.4 95.1) (width 0.2) (layer "F.Cu") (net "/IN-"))
 (segment (start 49.4 95.1) (end 51.5 93) (width 0.2) (layer "F.Cu") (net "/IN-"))
 (segment (start 19 95) (end 19.1 95.1) (width 0.2) (layer "F.Cu") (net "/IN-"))
 (segment (start 19.1 95.1) (end 49.4 95.1) (width 0.2) (layer "F.Cu") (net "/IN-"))
 (segment (start 49.4 56.6417) (end 42.2017 63.84) (width 0.2) (layer "F.Cu") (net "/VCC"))
 (segment (start 49.4 34.5) (end 49.4 56.6417) (width 0.2) (layer "F.Cu") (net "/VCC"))
 (segment (start 40.9 63.84) (end 42.2017 63.84) (width 0.2) (layer "F.Cu") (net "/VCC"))
 (segment (start 17.7035 32.4582) (end 56.9582 32.4582) (width 0.2) (layer "B.Cu") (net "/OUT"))
 (segment (start 16.8017 33.36) (end 17.7035 32.4582) (width 0.2) (layer "B.Cu") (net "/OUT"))
 (segment (start 15.5 33.36) (end 16.8017 33.36) (width 0.2) (layer "B.Cu") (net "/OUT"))
 (segment (start 56.9582 32.4582) (end 59 34.5) (width 0.2) (layer "B.Cu") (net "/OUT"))
 (segment (start 57.747 69.713) (end 57.747 35.9961) (width 0.2) (layer "F.Cu") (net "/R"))
 (segment (start 56 71.46) (end 57.747 69.713) (width 0.2) (layer "F.Cu") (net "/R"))
 (segment (start 56.6001 34.8492) (end 56.6001 31.7001) (width 0.2) (layer "F.Cu") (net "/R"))
 (segment (start 57.747 35.9961) (end 56.6001 34.8492) (width 0.2) (layer "F.Cu") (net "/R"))
 (segment (start 56.6001 31.7001) (end 54.4 29.5) (width 0.2) (layer "F.Cu") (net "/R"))
 (segment (start 15.5 51.14) (end 16.8017 51.14) (width 0.2) (layer "F.Cu") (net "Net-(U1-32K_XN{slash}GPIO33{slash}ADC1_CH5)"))
 (segment (start 28.0736 62.4119) (end 28.0736 92.8464) (width 0.2) (layer "F.Cu") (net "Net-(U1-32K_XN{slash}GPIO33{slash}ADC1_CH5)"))
 (segment (start 16.8017 51.14) (end 28.0736 62.4119) (width 0.2) (layer "F.Cu") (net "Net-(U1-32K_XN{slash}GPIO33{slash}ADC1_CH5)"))
 (segment (start 28.0736 92.8464) (end 26.92 94) (width 0.2) (layer "F.Cu") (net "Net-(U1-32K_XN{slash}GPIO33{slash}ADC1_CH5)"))
 (segment (start 15.0293 57.49) (end 15.9147 57.49) (width 0.2) (layer "F.Cu") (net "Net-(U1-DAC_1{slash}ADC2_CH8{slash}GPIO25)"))
 (segment (start 14.1983 56.659) (end 15.0293 57.49) (width 0.2) (layer "F.Cu") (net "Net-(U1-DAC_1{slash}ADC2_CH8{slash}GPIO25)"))
 (segment (start 21.0502 62.6255) (end 21.0502 84.1302) (width 0.2) (layer "F.Cu") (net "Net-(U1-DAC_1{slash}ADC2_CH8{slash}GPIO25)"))
 (segment (start 15.9147 57.49) (end 21.0502 62.6255) (width 0.2) (layer "F.Cu") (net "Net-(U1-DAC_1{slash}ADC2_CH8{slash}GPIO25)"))
 (segment (start 21.0502 84.1302) (end 26.92 90) (width 0.2) (layer "F.Cu") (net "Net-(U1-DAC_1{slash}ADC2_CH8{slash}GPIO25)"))
 (segment (start 14.1983 53.68) (end 14.1983 56.659) (width 0.2) (layer "F.Cu") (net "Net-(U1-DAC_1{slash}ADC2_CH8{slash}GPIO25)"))
 (segment (start 15.5 53.68) (end 14.1983 53.68) (width 0.2) (layer "F.Cu") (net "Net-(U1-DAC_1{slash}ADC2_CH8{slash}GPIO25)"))
 (segment (start 51.5 88) (end 25.7217 88) (width 0.2) (layer "B.Cu") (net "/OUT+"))
 (segment (start 25.7217 88) (end 16.8017 79.08) (width 0.2) (layer "B.Cu") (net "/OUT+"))
 (segment (start 15.5 79.08) (end 16.8017 79.08) (width 0.2) (layer "B.Cu") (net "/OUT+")))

